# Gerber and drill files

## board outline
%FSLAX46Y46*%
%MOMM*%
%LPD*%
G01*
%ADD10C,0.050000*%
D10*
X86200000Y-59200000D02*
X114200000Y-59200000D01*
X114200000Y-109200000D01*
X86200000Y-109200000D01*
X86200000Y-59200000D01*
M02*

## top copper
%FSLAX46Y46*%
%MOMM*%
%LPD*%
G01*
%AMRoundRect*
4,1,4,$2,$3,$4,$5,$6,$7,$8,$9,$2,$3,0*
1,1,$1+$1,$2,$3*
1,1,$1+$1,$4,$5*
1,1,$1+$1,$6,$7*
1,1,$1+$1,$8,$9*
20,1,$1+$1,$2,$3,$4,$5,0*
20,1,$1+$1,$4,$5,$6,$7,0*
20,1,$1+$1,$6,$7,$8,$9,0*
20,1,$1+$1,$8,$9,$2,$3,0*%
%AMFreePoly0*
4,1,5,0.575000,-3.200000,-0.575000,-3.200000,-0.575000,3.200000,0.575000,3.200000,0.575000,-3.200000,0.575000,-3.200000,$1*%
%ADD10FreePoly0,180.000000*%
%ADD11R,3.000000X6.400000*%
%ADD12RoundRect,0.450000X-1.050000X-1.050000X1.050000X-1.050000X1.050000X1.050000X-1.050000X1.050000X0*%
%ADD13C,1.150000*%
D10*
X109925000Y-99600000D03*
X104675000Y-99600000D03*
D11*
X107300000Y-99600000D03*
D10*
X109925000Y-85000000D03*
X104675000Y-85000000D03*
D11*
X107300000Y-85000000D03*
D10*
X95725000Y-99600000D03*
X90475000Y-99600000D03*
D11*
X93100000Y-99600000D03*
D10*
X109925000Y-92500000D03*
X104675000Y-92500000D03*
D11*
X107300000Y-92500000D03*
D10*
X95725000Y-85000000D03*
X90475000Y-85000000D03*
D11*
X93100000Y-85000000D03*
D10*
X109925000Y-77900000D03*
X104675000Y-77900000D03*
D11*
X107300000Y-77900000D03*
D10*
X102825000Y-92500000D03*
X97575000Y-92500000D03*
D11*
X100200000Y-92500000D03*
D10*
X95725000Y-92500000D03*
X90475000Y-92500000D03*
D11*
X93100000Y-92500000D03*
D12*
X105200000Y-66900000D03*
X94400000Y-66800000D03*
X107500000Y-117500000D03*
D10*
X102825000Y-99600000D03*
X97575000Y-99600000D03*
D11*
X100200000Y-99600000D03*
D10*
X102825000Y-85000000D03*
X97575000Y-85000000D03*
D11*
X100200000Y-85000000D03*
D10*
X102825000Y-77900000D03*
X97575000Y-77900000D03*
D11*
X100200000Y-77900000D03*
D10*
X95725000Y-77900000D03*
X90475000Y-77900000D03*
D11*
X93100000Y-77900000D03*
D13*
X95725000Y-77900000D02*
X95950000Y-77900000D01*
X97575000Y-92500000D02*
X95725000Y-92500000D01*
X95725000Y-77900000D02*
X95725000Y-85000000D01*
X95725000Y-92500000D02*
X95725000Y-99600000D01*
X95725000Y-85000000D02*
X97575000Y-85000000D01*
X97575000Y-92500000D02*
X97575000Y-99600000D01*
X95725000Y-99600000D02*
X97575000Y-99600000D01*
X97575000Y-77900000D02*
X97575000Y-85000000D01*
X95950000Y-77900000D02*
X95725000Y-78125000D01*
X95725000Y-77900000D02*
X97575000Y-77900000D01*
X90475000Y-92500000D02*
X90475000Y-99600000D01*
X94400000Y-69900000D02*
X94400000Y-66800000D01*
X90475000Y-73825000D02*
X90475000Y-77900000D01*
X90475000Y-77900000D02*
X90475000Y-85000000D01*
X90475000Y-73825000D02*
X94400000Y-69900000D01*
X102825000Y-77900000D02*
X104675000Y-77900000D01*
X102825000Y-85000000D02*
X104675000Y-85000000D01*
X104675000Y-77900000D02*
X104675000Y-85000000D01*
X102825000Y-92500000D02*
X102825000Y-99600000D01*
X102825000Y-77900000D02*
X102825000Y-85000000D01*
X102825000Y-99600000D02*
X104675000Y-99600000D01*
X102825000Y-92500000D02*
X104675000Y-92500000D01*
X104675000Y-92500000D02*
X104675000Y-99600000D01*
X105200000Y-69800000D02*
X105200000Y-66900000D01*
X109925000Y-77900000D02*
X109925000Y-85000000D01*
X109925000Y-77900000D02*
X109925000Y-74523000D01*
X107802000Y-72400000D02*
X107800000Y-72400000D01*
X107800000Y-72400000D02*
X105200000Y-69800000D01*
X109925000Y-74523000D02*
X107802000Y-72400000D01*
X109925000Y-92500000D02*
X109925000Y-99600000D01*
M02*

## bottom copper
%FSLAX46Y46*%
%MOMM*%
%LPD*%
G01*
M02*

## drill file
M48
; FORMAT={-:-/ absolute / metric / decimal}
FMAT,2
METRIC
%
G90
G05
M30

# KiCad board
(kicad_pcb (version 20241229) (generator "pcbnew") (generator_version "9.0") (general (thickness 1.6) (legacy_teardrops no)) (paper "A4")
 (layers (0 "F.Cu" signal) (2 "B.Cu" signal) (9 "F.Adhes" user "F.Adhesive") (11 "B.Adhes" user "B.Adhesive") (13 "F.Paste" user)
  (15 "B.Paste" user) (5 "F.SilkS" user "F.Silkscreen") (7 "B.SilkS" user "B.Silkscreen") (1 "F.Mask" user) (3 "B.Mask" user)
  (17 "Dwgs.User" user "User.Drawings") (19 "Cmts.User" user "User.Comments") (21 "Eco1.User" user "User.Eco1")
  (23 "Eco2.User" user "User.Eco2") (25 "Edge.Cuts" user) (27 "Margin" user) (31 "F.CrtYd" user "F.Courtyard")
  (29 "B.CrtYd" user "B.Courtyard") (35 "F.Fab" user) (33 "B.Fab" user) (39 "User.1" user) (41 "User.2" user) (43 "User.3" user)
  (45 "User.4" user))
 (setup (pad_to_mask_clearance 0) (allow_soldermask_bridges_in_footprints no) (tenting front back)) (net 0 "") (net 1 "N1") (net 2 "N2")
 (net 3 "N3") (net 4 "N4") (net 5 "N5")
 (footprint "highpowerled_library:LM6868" (layer "F.Cu") (at 110.5 96.4 180)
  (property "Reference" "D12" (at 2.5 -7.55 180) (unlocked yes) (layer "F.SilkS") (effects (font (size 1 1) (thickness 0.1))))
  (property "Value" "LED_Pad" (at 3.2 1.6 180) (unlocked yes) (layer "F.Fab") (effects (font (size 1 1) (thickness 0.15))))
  (pad "1" smd custom (at 0.575 -3.2 180) (size 1.15 6.4) (layers "F.Cu" "F.Mask" "F.Paste") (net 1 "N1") (clearance 0.075)
   (thermal_bridge_angle 45) (options (clearance outline) (anchor rect)) (primitives))
  (pad "2" smd custom (at 5.825 -3.2 180) (size 1.15 6.4) (layers "F.Cu" "F.Mask" "F.Paste") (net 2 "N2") (clearance 0.075)
   (thermal_bridge_angle 45) (options (clearance outline) (anchor rect)) (primitives))
  (pad "3" smd rect (at 3.2 -3.2 180) (size 3 6.4) (layers "F.Cu" "F.Mask" "F.Paste") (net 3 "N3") (clearance 0.075)
   (thermal_bridge_angle 45)))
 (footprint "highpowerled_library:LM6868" (layer "F.Cu") (at 110.5 81.8 180)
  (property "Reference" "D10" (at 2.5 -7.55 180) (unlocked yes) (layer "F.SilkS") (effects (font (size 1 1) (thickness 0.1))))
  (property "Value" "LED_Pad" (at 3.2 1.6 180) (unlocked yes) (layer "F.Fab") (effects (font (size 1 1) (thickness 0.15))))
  (pad "1" smd custom (at 0.575 -3.2 180) (size 1.15 6.4) (layers "F.Cu" "F.Mask" "F.Paste") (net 1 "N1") (clearance 0.075)
   (thermal_bridge_angle 45) (options (clearance outline) (anchor rect)) (primitives))
  (pad "2" smd custom (at 5.825 -3.2 180) (size 1.15 6.4) (layers "F.Cu" "F.Mask" "F.Paste") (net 2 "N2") (clearance 0.075)
   (thermal_bridge_angle 45) (options (clearance outline) (anchor rect)) (primitives))
  (pad "3" smd rect (at 3.2 -3.2 180) (size 3 6.4) (layers "F.Cu" "F.Mask" "F.Paste") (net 3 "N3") (clearance 0.075)
   (thermal_bridge_angle 45)))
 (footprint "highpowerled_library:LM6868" (layer "F.Cu") (at 96.3 96.4 180)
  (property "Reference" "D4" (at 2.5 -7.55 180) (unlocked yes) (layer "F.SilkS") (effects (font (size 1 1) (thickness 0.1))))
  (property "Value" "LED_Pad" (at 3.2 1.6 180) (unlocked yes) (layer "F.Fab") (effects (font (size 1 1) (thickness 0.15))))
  (pad "1" smd custom (at 0.575 -3.2 180) (size 1.15 6.4) (layers "F.Cu" "F.Mask" "F.Paste") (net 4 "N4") (clearance 0.075)
   (thermal_bridge_angle 45) (options (clearance outline) (anchor rect)) (primitives))
  (pad "2" smd custom (at 5.825 -3.2 180) (size 1.15 6.4) (layers "F.Cu" "F.Mask" "F.Paste") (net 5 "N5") (clearance 0.075)
   (thermal_bridge_angle 45) (options (clearance outline) (anchor rect)) (primitives))
  (pad "3" smd rect (at 3.2 -3.2 180) (size 3 6.4) (layers "F.Cu" "F.Mask" "F.Paste") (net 3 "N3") (clearance 0.075)
   (thermal_bridge_angle 45)))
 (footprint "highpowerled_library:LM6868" (layer "F.Cu") (at 110.5 89.3 180)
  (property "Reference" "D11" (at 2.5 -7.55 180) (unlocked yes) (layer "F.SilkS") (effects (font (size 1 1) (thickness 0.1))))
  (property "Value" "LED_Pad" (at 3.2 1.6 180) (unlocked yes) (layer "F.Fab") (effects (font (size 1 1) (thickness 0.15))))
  (pad "1" smd custom (at 0.575 -3.2 180) (size 1.15 6.4) (layers "F.Cu" "F.Mask" "F.Paste") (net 1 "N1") (clearance 0.075)
   (thermal_bridge_angle 45) (options (clearance outline) (anchor rect)) (primitives))
  (pad "2" smd custom (at 5.825 -3.2 180) (size 1.15 6.4) (layers "F.Cu" "F.Mask" "F.Paste") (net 2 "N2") (clearance 0.075)
   (thermal_bridge_angle 45) (options (clearance outline) (anchor rect)) (primitives))
  (pad "3" smd rect (at 3.2 -3.2 180) (size 3 6.4) (layers "F.Cu" "F.Mask" "F.Paste") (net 3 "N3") (clearance 0.075)
   (thermal_bridge_angle 45)))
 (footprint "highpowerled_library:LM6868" (layer "F.Cu") (at 96.3 81.8 180)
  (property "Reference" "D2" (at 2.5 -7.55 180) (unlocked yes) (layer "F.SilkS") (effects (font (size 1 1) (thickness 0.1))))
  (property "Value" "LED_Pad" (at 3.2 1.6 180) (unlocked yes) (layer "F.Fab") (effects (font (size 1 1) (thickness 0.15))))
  (pad "1" smd custom (at 0.575 -3.2 180) (size 1.15 6.4) (layers "F.Cu" "F.Mask" "F.Paste") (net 4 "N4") (clearance 0.075)
   (thermal_bridge_angle 45) (options (clearance outline) (anchor rect)) (primitives))
  (pad "2" smd custom (at 5.825 -3.2 180) (size 1.15 6.4) (layers "F.Cu" "F.Mask" "F.Paste") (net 5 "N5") (clearance 0.075)
   (thermal_bridge_angle 45) (options (clearance outline) (anchor rect)) (primitives))
  (pad "3" smd rect (at 3.2 -3.2 180) (size 3 6.4) (layers "F.Cu" "F.Mask" "F.Paste") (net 3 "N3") (clearance 0.075)
   (thermal_bridge_angle 45)))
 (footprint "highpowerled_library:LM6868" (layer "F.Cu") (at 110.5 74.7 180)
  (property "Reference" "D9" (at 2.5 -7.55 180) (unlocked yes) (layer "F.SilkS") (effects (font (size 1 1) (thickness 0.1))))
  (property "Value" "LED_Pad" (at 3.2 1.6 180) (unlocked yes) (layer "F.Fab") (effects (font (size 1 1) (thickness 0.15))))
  (pad "1" smd custom (at 0.575 -3.2 180) (size 1.15 6.4) (layers "F.Cu" "F.Mask" "F.Paste") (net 1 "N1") (clearance 0.075)
   (thermal_bridge_angle 45) (options (clearance outline) (anchor rect)) (primitives))
  (pad "2" smd custom (at 5.825 -3.2 180) (size 1.15 6.4) (layers "F.Cu" "F.Mask" "F.Paste") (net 2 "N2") (clearance 0.075)
   (thermal_bridge_angle 45) (options (clearance outline) (anchor rect)) (primitives))
  (pad "3" smd rect (at 3.2 -3.2 180) (size 3 6.4) (layers "F.Cu" "F.Mask" "F.Paste") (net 3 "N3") (clearance 0.075)
   (thermal_bridge_angle 45)))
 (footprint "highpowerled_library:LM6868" (layer "F.Cu") (at 103.4 89.3 180)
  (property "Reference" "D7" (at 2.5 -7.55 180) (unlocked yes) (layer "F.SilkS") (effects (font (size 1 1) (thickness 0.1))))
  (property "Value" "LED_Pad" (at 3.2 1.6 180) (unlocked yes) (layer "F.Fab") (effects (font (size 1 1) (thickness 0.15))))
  (pad "1" smd custom (at 0.575 -3.2 180) (size 1.15 6.4) (layers "F.Cu" "F.Mask" "F.Paste") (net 2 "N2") (clearance 0.075)
   (thermal_bridge_angle 45) (options (clearance outline) (anchor rect)) (primitives))
  (pad "2" smd custom (at 5.825 -3.2 180) (size 1.15 6.4) (layers "F.Cu" "F.Mask" "F.Paste") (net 4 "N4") (clearance 0.075)
   (thermal_bridge_angle 45) (options (clearance outline) (anchor rect)) (primitives))
  (pad "3" smd rect (at 3.2 -3.2 180) (size 3 6.4) (layers "F.Cu" "F.Mask" "F.Paste") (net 3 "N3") (clearance 0.075)
   (thermal_bridge_angle 45)))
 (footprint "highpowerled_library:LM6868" (layer "F.Cu") (at 96.3 89.3 180)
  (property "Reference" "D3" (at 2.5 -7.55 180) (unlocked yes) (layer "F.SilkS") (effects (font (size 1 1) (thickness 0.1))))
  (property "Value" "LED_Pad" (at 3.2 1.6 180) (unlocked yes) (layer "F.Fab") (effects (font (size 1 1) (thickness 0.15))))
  (pad "1" smd custom (at 0.575 -3.2 180) (size 1.15 6.4) (layers "F.Cu" "F.Mask" "F.Paste") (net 4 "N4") (clearance 0.075)
   (thermal_bridge_angle 45) (options (clearance outline) (anchor rect)) (primitives))
  (pad "2" smd custom (at 5.825 -3.2 180) (size 1.15 6.4) (layers "F.Cu" "F.Mask" "F.Paste") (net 5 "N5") (clearance 0.075)
   (thermal_bridge_angle 45) (options (clearance outline) (anchor rect)) (primitives))
  (pad "3" smd rect (at 3.2 -3.2 180) (size 3 6.4) (layers "F.Cu" "F.Mask" "F.Paste") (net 3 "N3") (clearance 0.075)
   (thermal_bridge_angle 45)))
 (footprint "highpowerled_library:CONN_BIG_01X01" (layer "F.Cu") (at 105.2 66.9)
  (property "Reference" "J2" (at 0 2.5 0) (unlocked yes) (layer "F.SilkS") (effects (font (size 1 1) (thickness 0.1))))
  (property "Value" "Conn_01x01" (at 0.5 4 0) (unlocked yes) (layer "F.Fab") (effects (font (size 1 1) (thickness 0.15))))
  (pad "1" smd roundrect (at 0 0) (size 3 3) (layers "F.Cu" "F.Mask" "F.Paste") (roundrect_rratio 0.15) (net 1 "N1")
   (thermal_bridge_angle 45)))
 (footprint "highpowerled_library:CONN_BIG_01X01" (layer "F.Cu") (at 94.4 66.8)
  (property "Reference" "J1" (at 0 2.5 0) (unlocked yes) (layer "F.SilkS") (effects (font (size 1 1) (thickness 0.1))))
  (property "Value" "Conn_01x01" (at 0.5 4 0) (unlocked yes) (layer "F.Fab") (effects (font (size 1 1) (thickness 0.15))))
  (pad "1" smd roundrect (at 0 0) (size 3 3) (layers "F.Cu" "F.Mask" "F.Paste") (roundrect_rratio 0.15) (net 5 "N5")
   (thermal_bridge_angle 45)))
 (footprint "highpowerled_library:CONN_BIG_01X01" (layer "F.Cu") (at 107.5 117.5)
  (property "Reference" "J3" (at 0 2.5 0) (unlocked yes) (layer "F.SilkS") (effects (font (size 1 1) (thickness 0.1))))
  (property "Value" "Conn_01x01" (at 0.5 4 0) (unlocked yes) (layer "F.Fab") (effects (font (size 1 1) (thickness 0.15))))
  (pad "1" smd roundrect (at 0 0) (size 3 3) (layers "F.Cu" "F.Mask" "F.Paste") (roundrect_rratio 0.15) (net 3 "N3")
   (thermal_bridge_angle 45)))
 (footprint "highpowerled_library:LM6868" (layer "F.Cu") (at 103.4 96.4 180)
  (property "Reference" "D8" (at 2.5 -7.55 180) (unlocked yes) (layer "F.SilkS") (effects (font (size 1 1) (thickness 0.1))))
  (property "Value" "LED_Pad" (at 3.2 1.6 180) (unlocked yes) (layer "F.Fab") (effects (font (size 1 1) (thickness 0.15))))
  (pad "1" smd custom (at 0.575 -3.2 180) (size 1.15 6.4) (layers "F.Cu" "F.Mask" "F.Paste") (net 2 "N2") (clearance 0.075)
   (thermal_bridge_angle 45) (options (clearance outline) (anchor rect)) (primitives))
  (pad "2" smd custom (at 5.825 -3.2 180) (size 1.15 6.4) (layers "F.Cu" "F.Mask" "F.Paste") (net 4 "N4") (clearance 0.075)
   (thermal_bridge_angle 45) (options (clearance outline) (anchor rect)) (primitives))
  (pad "3" smd rect (at 3.2 -3.2 180) (size 3 6.4) (layers "F.Cu" "F.Mask" "F.Paste") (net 3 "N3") (clearance 0.075)
   (thermal_bridge_angle 45)))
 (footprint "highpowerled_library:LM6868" (layer "F.Cu") (at 103.4 81.8 180)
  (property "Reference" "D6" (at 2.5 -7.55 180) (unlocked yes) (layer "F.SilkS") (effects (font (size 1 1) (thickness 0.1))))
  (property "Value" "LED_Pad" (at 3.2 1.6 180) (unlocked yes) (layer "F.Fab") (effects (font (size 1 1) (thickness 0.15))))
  (pad "1" smd custom (at 0.575 -3.2 180) (size 1.15 6.4) (layers "F.Cu" "F.Mask" "F.Paste") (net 2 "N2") (clearance 0.075)
   (thermal_bridge_angle 45) (options (clearance outline) (anchor rect)) (primitives))
  (pad "2" smd custom (at 5.825 -3.2 180) (size 1.15 6.4) (layers "F.Cu" "F.Mask" "F.Paste") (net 4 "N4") (clearance 0.075)
   (thermal_bridge_angle 45) (options (clearance outline) (anchor rect)) (primitives))
  (pad "3" smd rect (at 3.2 -3.2 180) (size 3 6.4) (layers "F.Cu" "F.Mask" "F.Paste") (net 3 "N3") (clearance 0.075)
   (thermal_bridge_angle 45)))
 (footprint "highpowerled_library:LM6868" (layer "F.Cu") (at 103.4 74.7 180)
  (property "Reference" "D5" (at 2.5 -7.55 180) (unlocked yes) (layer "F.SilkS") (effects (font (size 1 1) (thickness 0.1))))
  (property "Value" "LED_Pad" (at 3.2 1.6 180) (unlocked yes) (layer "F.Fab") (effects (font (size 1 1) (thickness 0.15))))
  (pad "1" smd custom (at 0.575 -3.2 180) (size 1.15 6.4) (layers "F.Cu" "F.Mask" "F.Paste") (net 2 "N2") (clearance 0.075)
   (thermal_bridge_angle 45) (options (clearance outline) (anchor rect)) (primitives))
  (pad "2" smd custom (at 5.825 -3.2 180) (size 1.15 6.4) (layers "F.Cu" "F.Mask" "F.Paste") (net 4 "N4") (clearance 0.075)
   (thermal_bridge_angle 45) (options (clearance outline) (anchor rect)) (primitives))
  (pad "3" smd rect (at 3.2 -3.2 180) (size 3 6.4) (layers "F.Cu" "F.Mask" "F.Paste") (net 3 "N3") (clearance 0.075)
   (thermal_bridge_angle 45)))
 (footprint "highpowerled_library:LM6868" (layer "F.Cu") (at 96.3 74.7 180)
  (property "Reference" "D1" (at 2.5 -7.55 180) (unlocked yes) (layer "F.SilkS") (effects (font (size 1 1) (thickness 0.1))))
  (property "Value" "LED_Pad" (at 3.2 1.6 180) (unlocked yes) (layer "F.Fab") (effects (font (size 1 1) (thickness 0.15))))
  (pad "1" smd custom (at 0.575 -3.2 180) (size 1.15 6.4) (layers "F.Cu" "F.Mask" "F.Paste") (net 4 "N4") (clearance 0.075)
   (thermal_bridge_angle 45) (options (clearance outline) (anchor rect)) (primitives))
  (pad "2" smd custom (at 5.825 -3.2 180) (size 1.15 6.4) (layers "F.Cu" "F.Mask" "F.Paste") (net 5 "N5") (clearance 0.075)
   (thermal_bridge_angle 45) (options (clearance outline) (anchor rect)) (primitives))
  (pad "3" smd rect (at 3.2 -3.2 180) (size 3 6.4) (layers "F.Cu" "F.Mask" "F.Paste") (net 3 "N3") (clearance 0.075)
   (thermal_bridge_angle 45)))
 (gr_rect (start 86.2 59.2) (end 114.2 109.2) (stroke (width 0.05) (type default)) (fill no) (layer "Edge.Cuts"))
 (segment (start 95.725 77.9) (end 95.95 77.9) (width 1.15) (layer "F.Cu") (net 4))
 (segment (start 97.575 92.5) (end 95.725 92.5) (width 1.15) (layer "F.Cu") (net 4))
 (segment (start 95.725 77.9) (end 95.725 85) (width 1.15) (layer "F.Cu") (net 4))
 (segment (start 95.725 92.5) (end 95.725 99.6) (width 1.15) (layer "F.Cu") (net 4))
 (segment (start 95.725 85) (end 97.575 85) (width 1.15) (layer "F.Cu") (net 4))
 (segment (start 97.575 92.5) (end 97.575 99.6) (width 1.15) (layer "F.Cu") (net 4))
 (segment (start 95.725 99.6) (end 97.575 99.6) (width 1.15) (layer "F.Cu") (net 4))
 (segment (start 97.575 77.9) (end 97.575 85) (width 1.15) (layer "F.Cu") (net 4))
 (segment (start 95.95 77.9) (end 95.725 78.125) (width 1.15) (layer "F.Cu") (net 4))
 (segment (start 95.725 77.9) (end 97.575 77.9) (width 1.15) (layer "F.Cu") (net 4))
 (segment (start 90.475 92.5) (end 90.475 99.6) (width 1.15) (layer "F.Cu") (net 5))
 (segment (start 94.4 69.9) (end 94.4 66.8) (width 1.15) (layer "F.Cu") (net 5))
 (segment (start 90.475 73.825) (end 90.475 77.9) (width 1.15) (layer "F.Cu") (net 5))
 (segment (start 90.475 77.9) (end 90.475 85) (width 1.15) (layer "F.Cu") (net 5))
 (segment (start 90.475 73.825) (end 94.4 69.9) (width 1.15) (layer "F.Cu") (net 5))
 (segment (start 102.825 77.9) (end 104.675 77.9) (width 1.15) (layer "F.Cu") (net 2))
 (segment (start 102.825 85) (end 104.675 85) (width 1.15) (layer "F.Cu") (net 2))
 (segment (start 104.675 77.9) (end 104.675 85) (width 1.15) (layer "F.Cu") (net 2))
 (segment (start 102.825 92.5) (end 102.825 99.6) (width 1.15) (layer "F.Cu") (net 2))
 (segment (start 102.825 77.9) (end 102.825 85) (width 1.15) (layer "F.Cu") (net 2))
 (segment (start 102.825 99.6) (end 104.675 99.6) (width 1.15) (layer "F.Cu") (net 2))
 (segment (start 102.825 92.5) (end 104.675 92.5) (width 1.15) (layer "F.Cu") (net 2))
 (segment (start 104.675 92.5) (end 104.675 99.6) (width 1.15) (layer "F.Cu") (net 2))
 (segment (start 105.2 69.8) (end 105.2 66.9) (width 1.15) (layer "F.Cu") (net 1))
 (segment (start 109.925 77.9) (end 109.925 85) (width 1.15) (layer "F.Cu") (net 1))
 (segment (start 109.925 77.9) (end 109.925 74.523) (width 1.15) (layer "F.Cu") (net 1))
 (segment (start 107.802 72.4) (end 107.8 72.4) (width 1.15) (layer "F.Cu") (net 1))
 (segment (start 107.8 72.4) (end 105.2 69.8) (width 1.15) (layer "F.Cu") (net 1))
 (segment (start 109.925 74.523) (end 107.802 72.4) (width 1.15) (layer "F.Cu") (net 1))
 (segment (start 109.925 92.5) (end 109.925 99.6) (width 1.15) (layer "F.Cu") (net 1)))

